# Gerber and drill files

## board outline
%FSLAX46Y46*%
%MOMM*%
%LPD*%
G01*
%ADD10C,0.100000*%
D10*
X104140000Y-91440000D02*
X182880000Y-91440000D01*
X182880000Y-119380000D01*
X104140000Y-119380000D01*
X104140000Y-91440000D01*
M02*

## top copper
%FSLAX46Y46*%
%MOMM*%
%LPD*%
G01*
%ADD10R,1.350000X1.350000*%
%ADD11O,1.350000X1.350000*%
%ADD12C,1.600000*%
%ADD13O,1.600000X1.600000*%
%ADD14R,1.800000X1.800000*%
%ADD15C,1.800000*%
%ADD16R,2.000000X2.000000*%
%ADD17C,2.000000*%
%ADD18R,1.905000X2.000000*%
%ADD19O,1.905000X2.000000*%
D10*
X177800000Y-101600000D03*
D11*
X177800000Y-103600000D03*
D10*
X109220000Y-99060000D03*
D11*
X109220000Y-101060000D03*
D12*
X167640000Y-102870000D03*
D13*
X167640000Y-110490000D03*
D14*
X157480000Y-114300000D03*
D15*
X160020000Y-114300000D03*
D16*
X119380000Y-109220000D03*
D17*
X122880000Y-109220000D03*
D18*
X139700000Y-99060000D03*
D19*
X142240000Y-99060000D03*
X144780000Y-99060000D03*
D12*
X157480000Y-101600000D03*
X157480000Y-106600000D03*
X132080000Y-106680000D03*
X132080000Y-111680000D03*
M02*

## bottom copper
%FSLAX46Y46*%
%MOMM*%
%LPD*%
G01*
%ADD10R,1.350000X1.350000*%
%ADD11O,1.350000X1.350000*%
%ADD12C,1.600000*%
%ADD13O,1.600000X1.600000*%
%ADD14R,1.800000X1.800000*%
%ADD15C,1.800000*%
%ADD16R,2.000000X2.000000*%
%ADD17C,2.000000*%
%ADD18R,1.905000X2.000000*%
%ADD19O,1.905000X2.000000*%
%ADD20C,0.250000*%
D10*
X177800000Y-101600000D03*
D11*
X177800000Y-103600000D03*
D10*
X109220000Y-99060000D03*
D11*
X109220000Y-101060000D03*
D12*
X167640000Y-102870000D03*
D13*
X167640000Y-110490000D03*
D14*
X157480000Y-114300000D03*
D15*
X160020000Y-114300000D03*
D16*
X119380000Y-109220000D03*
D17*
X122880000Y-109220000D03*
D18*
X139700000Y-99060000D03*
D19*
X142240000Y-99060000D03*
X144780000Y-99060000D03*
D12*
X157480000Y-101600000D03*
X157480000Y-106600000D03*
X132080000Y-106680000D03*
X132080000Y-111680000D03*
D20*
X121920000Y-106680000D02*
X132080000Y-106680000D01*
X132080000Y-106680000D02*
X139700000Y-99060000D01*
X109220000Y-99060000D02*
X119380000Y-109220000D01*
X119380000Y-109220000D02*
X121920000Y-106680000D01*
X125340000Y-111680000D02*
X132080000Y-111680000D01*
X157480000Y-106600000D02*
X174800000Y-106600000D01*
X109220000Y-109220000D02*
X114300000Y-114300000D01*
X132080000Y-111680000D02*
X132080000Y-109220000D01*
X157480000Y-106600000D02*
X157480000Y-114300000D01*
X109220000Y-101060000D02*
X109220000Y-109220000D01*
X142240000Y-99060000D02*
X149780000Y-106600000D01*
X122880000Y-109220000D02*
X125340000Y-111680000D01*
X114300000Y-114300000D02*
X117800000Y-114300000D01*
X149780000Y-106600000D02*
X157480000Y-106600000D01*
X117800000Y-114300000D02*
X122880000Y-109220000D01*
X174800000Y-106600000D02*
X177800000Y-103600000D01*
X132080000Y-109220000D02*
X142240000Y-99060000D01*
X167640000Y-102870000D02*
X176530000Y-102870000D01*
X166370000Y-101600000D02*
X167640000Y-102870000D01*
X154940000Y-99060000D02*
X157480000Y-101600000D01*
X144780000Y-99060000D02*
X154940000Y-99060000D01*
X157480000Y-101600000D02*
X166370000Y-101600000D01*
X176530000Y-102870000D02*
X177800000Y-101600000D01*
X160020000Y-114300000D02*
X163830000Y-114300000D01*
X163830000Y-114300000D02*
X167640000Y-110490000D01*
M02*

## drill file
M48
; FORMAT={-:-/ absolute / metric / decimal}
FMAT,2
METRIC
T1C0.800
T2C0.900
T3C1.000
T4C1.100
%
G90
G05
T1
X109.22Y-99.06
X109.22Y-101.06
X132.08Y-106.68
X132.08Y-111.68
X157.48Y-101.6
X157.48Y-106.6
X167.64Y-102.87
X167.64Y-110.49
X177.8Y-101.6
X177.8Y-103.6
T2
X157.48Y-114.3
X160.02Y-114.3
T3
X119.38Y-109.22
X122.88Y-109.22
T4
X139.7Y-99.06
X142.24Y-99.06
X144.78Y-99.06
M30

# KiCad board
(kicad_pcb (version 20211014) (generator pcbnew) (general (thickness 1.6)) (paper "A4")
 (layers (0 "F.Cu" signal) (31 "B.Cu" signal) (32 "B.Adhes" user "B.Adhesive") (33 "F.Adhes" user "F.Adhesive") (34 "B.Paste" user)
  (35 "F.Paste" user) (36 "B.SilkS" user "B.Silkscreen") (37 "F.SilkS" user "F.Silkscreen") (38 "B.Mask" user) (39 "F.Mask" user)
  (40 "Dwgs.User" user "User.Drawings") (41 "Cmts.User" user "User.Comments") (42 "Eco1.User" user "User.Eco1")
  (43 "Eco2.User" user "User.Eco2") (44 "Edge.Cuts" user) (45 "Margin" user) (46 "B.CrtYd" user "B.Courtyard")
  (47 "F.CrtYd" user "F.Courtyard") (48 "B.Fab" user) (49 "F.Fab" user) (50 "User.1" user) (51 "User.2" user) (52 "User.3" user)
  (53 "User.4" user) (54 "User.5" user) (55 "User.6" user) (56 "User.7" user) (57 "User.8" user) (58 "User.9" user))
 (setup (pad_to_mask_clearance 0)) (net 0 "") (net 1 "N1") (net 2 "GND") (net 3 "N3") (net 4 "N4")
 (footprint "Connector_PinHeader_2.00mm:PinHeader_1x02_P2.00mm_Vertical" (layer "F.Cu") (at 177.8 101.6)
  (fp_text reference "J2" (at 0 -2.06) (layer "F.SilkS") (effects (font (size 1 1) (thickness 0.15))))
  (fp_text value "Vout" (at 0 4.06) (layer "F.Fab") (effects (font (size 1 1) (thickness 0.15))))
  (pad "1" thru_hole rect (at 0 0) (size 1.35 1.35) (drill 0.8) (layers *.Cu *.Mask) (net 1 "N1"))
  (pad "2" thru_hole oval (at 0 2) (size 1.35 1.35) (drill 0.8) (layers *.Cu *.Mask) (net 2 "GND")))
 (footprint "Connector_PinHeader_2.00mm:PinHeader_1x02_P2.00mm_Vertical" (layer "F.Cu") (at 109.22 99.06)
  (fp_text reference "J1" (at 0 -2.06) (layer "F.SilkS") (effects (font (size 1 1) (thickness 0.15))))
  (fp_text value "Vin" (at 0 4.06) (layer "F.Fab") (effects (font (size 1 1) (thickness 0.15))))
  (pad "1" thru_hole rect (at 0 0) (size 1.35 1.35) (drill 0.8) (layers *.Cu *.Mask) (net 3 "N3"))
  (pad "2" thru_hole oval (at 0 2) (size 1.35 1.35) (drill 0.8) (layers *.Cu *.Mask) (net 2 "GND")))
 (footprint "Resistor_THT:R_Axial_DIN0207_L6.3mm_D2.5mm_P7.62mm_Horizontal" (layer "F.Cu") (at 167.64 102.87 -90)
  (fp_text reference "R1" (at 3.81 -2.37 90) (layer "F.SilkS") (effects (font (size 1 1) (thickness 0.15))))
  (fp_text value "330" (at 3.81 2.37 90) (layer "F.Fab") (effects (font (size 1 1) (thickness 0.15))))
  (pad "1" thru_hole circle (at 0 0 270) (size 1.6 1.6) (drill 0.8) (layers *.Cu *.Mask) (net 1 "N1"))
  (pad "2" thru_hole oval (at 7.62 0 270) (size 1.6 1.6) (drill 0.8) (layers *.Cu *.Mask) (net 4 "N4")))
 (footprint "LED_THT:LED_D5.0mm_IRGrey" (layer "F.Cu") (at 157.48 114.3)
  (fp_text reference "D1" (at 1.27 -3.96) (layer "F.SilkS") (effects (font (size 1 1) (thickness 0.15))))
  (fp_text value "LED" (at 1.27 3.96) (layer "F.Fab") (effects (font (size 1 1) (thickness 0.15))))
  (pad "1" thru_hole rect (at 0 0) (size 1.8 1.8) (drill 0.9) (layers *.Cu *.Mask) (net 2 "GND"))
  (pad "2" thru_hole circle (at 2.54 0) (size 1.8 1.8) (drill 0.9) (layers *.Cu *.Mask) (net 4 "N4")))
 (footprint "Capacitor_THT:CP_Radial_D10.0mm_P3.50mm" (layer "F.Cu") (at 119.38 109.22)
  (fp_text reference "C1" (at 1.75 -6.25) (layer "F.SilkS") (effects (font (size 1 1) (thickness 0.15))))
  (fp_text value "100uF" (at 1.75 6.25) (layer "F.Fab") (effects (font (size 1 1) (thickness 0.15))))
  (pad "1" thru_hole rect (at 0 0) (size 2 2) (drill 1) (layers *.Cu *.Mask) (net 3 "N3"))
  (pad "2" thru_hole circle (at 3.5 0) (size 2 2) (drill 1) (layers *.Cu *.Mask) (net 2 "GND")))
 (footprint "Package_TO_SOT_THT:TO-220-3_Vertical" (layer "F.Cu") (at 139.7 99.06)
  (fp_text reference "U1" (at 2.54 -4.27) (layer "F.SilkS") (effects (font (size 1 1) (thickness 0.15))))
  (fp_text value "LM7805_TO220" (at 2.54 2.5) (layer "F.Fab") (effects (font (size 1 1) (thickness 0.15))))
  (pad "1" thru_hole rect (at 0 0) (size 1.905 2) (drill 1.1) (layers *.Cu *.Mask) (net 3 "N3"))
  (pad "2" thru_hole oval (at 2.54 0) (size 1.905 2) (drill 1.1) (layers *.Cu *.Mask) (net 2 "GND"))
  (pad "3" thru_hole oval (at 5.08 0) (size 1.905 2) (drill 1.1) (layers *.Cu *.Mask) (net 1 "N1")))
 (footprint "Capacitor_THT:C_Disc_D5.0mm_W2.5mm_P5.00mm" (layer "F.Cu") (at 157.48 101.6 -90)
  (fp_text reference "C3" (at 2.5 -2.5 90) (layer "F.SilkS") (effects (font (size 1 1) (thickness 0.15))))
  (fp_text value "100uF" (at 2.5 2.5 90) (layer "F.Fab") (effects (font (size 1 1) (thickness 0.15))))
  (pad "1" thru_hole circle (at 0 0 270) (size 1.6 1.6) (drill 0.8) (layers *.Cu *.Mask) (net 1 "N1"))
  (pad "2" thru_hole circle (at 5 0 270) (size 1.6 1.6) (drill 0.8) (layers *.Cu *.Mask) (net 2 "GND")))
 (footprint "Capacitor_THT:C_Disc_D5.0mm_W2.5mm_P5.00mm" (layer "F.Cu") (at 132.08 106.68 -90)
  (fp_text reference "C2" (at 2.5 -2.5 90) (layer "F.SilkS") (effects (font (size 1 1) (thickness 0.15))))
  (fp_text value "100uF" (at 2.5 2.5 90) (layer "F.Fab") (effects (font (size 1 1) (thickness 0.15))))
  (pad "1" thru_hole circle (at 0 0 270) (size 1.6 1.6) (drill 0.8) (layers *.Cu *.Mask) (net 3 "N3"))
  (pad "2" thru_hole circle (at 5 0 270) (size 1.6 1.6) (drill 0.8) (layers *.Cu *.Mask) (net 2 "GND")))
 (gr_rect (start 182.88 119.38) (end 104.14 91.44) (layer "Edge.Cuts") (width 0.1) (fill none))
 (segment (start 121.92 106.68) (end 132.08 106.68) (width 0.25) (layer "B.Cu") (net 3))
 (segment (start 132.08 106.68) (end 139.7 99.06) (width 0.25) (layer "B.Cu") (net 3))
 (segment (start 109.22 99.06) (end 119.38 109.22) (width 0.25) (layer "B.Cu") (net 3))
 (segment (start 119.38 109.22) (end 121.92 106.68) (width 0.25) (layer "B.Cu") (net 3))
 (segment (start 125.34 111.68) (end 132.08 111.68) (width 0.25) (layer "B.Cu") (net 2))
 (segment (start 157.48 106.6) (end 174.8 106.6) (width 0.25) (layer "B.Cu") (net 2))
 (segment (start 109.22 109.22) (end 114.3 114.3) (width 0.25) (layer "B.Cu") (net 2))
 (segment (start 132.08 111.68) (end 132.08 109.22) (width 0.25) (layer "B.Cu") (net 2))
 (segment (start 157.48 106.6) (end 157.48 114.3) (width 0.25) (layer "B.Cu") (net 2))
 (segment (start 109.22 101.06) (end 109.22 109.22) (width 0.25) (layer "B.Cu") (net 2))
 (segment (start 142.24 99.06) (end 149.78 106.6) (width 0.25) (layer "B.Cu") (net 2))
 (segment (start 122.88 109.22) (end 125.34 111.68) (width 0.25) (layer "B.Cu") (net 2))
 (segment (start 114.3 114.3) (end 117.8 114.3) (width 0.25) (layer "B.Cu") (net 2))
 (segment (start 149.78 106.6) (end 157.48 106.6) (width 0.25) (layer "B.Cu") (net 2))
 (segment (start 117.8 114.3) (end 122.88 109.22) (width 0.25) (layer "B.Cu") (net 2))
 (segment (start 174.8 106.6) (end 177.8 103.6) (width 0.25) (layer "B.Cu") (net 2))
 (segment (start 132.08 109.22) (end 142.24 99.06) (width 0.25) (layer "B.Cu") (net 2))
 (segment (start 167.64 102.87) (end 176.53 102.87) (width 0.25) (layer "B.Cu") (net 1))
 (segment (start 166.37 101.6) (end 167.64 102.87) (width 0.25) (layer "B.Cu") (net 1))
 (segment (start 154.94 99.06) (end 157.48 101.6) (width 0.25) (layer "B.Cu") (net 1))
 (segment (start 144.78 99.06) (end 154.94 99.06) (width 0.25) (layer "B.Cu") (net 1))
 (segment (start 157.48 101.6) (end 166.37 101.6) (width 0.25) (layer "B.Cu") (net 1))
 (segment (start 176.53 102.87) (end 177.8 101.6) (width 0.25) (layer "B.Cu") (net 1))
 (segment (start 160.02 114.3) (end 163.83 114.3) (width 0.25) (layer "B.Cu") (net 4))
 (segment (start 163.83 114.3) (end 167.64 110.49) (width 0.25) (layer "B.Cu") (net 4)))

